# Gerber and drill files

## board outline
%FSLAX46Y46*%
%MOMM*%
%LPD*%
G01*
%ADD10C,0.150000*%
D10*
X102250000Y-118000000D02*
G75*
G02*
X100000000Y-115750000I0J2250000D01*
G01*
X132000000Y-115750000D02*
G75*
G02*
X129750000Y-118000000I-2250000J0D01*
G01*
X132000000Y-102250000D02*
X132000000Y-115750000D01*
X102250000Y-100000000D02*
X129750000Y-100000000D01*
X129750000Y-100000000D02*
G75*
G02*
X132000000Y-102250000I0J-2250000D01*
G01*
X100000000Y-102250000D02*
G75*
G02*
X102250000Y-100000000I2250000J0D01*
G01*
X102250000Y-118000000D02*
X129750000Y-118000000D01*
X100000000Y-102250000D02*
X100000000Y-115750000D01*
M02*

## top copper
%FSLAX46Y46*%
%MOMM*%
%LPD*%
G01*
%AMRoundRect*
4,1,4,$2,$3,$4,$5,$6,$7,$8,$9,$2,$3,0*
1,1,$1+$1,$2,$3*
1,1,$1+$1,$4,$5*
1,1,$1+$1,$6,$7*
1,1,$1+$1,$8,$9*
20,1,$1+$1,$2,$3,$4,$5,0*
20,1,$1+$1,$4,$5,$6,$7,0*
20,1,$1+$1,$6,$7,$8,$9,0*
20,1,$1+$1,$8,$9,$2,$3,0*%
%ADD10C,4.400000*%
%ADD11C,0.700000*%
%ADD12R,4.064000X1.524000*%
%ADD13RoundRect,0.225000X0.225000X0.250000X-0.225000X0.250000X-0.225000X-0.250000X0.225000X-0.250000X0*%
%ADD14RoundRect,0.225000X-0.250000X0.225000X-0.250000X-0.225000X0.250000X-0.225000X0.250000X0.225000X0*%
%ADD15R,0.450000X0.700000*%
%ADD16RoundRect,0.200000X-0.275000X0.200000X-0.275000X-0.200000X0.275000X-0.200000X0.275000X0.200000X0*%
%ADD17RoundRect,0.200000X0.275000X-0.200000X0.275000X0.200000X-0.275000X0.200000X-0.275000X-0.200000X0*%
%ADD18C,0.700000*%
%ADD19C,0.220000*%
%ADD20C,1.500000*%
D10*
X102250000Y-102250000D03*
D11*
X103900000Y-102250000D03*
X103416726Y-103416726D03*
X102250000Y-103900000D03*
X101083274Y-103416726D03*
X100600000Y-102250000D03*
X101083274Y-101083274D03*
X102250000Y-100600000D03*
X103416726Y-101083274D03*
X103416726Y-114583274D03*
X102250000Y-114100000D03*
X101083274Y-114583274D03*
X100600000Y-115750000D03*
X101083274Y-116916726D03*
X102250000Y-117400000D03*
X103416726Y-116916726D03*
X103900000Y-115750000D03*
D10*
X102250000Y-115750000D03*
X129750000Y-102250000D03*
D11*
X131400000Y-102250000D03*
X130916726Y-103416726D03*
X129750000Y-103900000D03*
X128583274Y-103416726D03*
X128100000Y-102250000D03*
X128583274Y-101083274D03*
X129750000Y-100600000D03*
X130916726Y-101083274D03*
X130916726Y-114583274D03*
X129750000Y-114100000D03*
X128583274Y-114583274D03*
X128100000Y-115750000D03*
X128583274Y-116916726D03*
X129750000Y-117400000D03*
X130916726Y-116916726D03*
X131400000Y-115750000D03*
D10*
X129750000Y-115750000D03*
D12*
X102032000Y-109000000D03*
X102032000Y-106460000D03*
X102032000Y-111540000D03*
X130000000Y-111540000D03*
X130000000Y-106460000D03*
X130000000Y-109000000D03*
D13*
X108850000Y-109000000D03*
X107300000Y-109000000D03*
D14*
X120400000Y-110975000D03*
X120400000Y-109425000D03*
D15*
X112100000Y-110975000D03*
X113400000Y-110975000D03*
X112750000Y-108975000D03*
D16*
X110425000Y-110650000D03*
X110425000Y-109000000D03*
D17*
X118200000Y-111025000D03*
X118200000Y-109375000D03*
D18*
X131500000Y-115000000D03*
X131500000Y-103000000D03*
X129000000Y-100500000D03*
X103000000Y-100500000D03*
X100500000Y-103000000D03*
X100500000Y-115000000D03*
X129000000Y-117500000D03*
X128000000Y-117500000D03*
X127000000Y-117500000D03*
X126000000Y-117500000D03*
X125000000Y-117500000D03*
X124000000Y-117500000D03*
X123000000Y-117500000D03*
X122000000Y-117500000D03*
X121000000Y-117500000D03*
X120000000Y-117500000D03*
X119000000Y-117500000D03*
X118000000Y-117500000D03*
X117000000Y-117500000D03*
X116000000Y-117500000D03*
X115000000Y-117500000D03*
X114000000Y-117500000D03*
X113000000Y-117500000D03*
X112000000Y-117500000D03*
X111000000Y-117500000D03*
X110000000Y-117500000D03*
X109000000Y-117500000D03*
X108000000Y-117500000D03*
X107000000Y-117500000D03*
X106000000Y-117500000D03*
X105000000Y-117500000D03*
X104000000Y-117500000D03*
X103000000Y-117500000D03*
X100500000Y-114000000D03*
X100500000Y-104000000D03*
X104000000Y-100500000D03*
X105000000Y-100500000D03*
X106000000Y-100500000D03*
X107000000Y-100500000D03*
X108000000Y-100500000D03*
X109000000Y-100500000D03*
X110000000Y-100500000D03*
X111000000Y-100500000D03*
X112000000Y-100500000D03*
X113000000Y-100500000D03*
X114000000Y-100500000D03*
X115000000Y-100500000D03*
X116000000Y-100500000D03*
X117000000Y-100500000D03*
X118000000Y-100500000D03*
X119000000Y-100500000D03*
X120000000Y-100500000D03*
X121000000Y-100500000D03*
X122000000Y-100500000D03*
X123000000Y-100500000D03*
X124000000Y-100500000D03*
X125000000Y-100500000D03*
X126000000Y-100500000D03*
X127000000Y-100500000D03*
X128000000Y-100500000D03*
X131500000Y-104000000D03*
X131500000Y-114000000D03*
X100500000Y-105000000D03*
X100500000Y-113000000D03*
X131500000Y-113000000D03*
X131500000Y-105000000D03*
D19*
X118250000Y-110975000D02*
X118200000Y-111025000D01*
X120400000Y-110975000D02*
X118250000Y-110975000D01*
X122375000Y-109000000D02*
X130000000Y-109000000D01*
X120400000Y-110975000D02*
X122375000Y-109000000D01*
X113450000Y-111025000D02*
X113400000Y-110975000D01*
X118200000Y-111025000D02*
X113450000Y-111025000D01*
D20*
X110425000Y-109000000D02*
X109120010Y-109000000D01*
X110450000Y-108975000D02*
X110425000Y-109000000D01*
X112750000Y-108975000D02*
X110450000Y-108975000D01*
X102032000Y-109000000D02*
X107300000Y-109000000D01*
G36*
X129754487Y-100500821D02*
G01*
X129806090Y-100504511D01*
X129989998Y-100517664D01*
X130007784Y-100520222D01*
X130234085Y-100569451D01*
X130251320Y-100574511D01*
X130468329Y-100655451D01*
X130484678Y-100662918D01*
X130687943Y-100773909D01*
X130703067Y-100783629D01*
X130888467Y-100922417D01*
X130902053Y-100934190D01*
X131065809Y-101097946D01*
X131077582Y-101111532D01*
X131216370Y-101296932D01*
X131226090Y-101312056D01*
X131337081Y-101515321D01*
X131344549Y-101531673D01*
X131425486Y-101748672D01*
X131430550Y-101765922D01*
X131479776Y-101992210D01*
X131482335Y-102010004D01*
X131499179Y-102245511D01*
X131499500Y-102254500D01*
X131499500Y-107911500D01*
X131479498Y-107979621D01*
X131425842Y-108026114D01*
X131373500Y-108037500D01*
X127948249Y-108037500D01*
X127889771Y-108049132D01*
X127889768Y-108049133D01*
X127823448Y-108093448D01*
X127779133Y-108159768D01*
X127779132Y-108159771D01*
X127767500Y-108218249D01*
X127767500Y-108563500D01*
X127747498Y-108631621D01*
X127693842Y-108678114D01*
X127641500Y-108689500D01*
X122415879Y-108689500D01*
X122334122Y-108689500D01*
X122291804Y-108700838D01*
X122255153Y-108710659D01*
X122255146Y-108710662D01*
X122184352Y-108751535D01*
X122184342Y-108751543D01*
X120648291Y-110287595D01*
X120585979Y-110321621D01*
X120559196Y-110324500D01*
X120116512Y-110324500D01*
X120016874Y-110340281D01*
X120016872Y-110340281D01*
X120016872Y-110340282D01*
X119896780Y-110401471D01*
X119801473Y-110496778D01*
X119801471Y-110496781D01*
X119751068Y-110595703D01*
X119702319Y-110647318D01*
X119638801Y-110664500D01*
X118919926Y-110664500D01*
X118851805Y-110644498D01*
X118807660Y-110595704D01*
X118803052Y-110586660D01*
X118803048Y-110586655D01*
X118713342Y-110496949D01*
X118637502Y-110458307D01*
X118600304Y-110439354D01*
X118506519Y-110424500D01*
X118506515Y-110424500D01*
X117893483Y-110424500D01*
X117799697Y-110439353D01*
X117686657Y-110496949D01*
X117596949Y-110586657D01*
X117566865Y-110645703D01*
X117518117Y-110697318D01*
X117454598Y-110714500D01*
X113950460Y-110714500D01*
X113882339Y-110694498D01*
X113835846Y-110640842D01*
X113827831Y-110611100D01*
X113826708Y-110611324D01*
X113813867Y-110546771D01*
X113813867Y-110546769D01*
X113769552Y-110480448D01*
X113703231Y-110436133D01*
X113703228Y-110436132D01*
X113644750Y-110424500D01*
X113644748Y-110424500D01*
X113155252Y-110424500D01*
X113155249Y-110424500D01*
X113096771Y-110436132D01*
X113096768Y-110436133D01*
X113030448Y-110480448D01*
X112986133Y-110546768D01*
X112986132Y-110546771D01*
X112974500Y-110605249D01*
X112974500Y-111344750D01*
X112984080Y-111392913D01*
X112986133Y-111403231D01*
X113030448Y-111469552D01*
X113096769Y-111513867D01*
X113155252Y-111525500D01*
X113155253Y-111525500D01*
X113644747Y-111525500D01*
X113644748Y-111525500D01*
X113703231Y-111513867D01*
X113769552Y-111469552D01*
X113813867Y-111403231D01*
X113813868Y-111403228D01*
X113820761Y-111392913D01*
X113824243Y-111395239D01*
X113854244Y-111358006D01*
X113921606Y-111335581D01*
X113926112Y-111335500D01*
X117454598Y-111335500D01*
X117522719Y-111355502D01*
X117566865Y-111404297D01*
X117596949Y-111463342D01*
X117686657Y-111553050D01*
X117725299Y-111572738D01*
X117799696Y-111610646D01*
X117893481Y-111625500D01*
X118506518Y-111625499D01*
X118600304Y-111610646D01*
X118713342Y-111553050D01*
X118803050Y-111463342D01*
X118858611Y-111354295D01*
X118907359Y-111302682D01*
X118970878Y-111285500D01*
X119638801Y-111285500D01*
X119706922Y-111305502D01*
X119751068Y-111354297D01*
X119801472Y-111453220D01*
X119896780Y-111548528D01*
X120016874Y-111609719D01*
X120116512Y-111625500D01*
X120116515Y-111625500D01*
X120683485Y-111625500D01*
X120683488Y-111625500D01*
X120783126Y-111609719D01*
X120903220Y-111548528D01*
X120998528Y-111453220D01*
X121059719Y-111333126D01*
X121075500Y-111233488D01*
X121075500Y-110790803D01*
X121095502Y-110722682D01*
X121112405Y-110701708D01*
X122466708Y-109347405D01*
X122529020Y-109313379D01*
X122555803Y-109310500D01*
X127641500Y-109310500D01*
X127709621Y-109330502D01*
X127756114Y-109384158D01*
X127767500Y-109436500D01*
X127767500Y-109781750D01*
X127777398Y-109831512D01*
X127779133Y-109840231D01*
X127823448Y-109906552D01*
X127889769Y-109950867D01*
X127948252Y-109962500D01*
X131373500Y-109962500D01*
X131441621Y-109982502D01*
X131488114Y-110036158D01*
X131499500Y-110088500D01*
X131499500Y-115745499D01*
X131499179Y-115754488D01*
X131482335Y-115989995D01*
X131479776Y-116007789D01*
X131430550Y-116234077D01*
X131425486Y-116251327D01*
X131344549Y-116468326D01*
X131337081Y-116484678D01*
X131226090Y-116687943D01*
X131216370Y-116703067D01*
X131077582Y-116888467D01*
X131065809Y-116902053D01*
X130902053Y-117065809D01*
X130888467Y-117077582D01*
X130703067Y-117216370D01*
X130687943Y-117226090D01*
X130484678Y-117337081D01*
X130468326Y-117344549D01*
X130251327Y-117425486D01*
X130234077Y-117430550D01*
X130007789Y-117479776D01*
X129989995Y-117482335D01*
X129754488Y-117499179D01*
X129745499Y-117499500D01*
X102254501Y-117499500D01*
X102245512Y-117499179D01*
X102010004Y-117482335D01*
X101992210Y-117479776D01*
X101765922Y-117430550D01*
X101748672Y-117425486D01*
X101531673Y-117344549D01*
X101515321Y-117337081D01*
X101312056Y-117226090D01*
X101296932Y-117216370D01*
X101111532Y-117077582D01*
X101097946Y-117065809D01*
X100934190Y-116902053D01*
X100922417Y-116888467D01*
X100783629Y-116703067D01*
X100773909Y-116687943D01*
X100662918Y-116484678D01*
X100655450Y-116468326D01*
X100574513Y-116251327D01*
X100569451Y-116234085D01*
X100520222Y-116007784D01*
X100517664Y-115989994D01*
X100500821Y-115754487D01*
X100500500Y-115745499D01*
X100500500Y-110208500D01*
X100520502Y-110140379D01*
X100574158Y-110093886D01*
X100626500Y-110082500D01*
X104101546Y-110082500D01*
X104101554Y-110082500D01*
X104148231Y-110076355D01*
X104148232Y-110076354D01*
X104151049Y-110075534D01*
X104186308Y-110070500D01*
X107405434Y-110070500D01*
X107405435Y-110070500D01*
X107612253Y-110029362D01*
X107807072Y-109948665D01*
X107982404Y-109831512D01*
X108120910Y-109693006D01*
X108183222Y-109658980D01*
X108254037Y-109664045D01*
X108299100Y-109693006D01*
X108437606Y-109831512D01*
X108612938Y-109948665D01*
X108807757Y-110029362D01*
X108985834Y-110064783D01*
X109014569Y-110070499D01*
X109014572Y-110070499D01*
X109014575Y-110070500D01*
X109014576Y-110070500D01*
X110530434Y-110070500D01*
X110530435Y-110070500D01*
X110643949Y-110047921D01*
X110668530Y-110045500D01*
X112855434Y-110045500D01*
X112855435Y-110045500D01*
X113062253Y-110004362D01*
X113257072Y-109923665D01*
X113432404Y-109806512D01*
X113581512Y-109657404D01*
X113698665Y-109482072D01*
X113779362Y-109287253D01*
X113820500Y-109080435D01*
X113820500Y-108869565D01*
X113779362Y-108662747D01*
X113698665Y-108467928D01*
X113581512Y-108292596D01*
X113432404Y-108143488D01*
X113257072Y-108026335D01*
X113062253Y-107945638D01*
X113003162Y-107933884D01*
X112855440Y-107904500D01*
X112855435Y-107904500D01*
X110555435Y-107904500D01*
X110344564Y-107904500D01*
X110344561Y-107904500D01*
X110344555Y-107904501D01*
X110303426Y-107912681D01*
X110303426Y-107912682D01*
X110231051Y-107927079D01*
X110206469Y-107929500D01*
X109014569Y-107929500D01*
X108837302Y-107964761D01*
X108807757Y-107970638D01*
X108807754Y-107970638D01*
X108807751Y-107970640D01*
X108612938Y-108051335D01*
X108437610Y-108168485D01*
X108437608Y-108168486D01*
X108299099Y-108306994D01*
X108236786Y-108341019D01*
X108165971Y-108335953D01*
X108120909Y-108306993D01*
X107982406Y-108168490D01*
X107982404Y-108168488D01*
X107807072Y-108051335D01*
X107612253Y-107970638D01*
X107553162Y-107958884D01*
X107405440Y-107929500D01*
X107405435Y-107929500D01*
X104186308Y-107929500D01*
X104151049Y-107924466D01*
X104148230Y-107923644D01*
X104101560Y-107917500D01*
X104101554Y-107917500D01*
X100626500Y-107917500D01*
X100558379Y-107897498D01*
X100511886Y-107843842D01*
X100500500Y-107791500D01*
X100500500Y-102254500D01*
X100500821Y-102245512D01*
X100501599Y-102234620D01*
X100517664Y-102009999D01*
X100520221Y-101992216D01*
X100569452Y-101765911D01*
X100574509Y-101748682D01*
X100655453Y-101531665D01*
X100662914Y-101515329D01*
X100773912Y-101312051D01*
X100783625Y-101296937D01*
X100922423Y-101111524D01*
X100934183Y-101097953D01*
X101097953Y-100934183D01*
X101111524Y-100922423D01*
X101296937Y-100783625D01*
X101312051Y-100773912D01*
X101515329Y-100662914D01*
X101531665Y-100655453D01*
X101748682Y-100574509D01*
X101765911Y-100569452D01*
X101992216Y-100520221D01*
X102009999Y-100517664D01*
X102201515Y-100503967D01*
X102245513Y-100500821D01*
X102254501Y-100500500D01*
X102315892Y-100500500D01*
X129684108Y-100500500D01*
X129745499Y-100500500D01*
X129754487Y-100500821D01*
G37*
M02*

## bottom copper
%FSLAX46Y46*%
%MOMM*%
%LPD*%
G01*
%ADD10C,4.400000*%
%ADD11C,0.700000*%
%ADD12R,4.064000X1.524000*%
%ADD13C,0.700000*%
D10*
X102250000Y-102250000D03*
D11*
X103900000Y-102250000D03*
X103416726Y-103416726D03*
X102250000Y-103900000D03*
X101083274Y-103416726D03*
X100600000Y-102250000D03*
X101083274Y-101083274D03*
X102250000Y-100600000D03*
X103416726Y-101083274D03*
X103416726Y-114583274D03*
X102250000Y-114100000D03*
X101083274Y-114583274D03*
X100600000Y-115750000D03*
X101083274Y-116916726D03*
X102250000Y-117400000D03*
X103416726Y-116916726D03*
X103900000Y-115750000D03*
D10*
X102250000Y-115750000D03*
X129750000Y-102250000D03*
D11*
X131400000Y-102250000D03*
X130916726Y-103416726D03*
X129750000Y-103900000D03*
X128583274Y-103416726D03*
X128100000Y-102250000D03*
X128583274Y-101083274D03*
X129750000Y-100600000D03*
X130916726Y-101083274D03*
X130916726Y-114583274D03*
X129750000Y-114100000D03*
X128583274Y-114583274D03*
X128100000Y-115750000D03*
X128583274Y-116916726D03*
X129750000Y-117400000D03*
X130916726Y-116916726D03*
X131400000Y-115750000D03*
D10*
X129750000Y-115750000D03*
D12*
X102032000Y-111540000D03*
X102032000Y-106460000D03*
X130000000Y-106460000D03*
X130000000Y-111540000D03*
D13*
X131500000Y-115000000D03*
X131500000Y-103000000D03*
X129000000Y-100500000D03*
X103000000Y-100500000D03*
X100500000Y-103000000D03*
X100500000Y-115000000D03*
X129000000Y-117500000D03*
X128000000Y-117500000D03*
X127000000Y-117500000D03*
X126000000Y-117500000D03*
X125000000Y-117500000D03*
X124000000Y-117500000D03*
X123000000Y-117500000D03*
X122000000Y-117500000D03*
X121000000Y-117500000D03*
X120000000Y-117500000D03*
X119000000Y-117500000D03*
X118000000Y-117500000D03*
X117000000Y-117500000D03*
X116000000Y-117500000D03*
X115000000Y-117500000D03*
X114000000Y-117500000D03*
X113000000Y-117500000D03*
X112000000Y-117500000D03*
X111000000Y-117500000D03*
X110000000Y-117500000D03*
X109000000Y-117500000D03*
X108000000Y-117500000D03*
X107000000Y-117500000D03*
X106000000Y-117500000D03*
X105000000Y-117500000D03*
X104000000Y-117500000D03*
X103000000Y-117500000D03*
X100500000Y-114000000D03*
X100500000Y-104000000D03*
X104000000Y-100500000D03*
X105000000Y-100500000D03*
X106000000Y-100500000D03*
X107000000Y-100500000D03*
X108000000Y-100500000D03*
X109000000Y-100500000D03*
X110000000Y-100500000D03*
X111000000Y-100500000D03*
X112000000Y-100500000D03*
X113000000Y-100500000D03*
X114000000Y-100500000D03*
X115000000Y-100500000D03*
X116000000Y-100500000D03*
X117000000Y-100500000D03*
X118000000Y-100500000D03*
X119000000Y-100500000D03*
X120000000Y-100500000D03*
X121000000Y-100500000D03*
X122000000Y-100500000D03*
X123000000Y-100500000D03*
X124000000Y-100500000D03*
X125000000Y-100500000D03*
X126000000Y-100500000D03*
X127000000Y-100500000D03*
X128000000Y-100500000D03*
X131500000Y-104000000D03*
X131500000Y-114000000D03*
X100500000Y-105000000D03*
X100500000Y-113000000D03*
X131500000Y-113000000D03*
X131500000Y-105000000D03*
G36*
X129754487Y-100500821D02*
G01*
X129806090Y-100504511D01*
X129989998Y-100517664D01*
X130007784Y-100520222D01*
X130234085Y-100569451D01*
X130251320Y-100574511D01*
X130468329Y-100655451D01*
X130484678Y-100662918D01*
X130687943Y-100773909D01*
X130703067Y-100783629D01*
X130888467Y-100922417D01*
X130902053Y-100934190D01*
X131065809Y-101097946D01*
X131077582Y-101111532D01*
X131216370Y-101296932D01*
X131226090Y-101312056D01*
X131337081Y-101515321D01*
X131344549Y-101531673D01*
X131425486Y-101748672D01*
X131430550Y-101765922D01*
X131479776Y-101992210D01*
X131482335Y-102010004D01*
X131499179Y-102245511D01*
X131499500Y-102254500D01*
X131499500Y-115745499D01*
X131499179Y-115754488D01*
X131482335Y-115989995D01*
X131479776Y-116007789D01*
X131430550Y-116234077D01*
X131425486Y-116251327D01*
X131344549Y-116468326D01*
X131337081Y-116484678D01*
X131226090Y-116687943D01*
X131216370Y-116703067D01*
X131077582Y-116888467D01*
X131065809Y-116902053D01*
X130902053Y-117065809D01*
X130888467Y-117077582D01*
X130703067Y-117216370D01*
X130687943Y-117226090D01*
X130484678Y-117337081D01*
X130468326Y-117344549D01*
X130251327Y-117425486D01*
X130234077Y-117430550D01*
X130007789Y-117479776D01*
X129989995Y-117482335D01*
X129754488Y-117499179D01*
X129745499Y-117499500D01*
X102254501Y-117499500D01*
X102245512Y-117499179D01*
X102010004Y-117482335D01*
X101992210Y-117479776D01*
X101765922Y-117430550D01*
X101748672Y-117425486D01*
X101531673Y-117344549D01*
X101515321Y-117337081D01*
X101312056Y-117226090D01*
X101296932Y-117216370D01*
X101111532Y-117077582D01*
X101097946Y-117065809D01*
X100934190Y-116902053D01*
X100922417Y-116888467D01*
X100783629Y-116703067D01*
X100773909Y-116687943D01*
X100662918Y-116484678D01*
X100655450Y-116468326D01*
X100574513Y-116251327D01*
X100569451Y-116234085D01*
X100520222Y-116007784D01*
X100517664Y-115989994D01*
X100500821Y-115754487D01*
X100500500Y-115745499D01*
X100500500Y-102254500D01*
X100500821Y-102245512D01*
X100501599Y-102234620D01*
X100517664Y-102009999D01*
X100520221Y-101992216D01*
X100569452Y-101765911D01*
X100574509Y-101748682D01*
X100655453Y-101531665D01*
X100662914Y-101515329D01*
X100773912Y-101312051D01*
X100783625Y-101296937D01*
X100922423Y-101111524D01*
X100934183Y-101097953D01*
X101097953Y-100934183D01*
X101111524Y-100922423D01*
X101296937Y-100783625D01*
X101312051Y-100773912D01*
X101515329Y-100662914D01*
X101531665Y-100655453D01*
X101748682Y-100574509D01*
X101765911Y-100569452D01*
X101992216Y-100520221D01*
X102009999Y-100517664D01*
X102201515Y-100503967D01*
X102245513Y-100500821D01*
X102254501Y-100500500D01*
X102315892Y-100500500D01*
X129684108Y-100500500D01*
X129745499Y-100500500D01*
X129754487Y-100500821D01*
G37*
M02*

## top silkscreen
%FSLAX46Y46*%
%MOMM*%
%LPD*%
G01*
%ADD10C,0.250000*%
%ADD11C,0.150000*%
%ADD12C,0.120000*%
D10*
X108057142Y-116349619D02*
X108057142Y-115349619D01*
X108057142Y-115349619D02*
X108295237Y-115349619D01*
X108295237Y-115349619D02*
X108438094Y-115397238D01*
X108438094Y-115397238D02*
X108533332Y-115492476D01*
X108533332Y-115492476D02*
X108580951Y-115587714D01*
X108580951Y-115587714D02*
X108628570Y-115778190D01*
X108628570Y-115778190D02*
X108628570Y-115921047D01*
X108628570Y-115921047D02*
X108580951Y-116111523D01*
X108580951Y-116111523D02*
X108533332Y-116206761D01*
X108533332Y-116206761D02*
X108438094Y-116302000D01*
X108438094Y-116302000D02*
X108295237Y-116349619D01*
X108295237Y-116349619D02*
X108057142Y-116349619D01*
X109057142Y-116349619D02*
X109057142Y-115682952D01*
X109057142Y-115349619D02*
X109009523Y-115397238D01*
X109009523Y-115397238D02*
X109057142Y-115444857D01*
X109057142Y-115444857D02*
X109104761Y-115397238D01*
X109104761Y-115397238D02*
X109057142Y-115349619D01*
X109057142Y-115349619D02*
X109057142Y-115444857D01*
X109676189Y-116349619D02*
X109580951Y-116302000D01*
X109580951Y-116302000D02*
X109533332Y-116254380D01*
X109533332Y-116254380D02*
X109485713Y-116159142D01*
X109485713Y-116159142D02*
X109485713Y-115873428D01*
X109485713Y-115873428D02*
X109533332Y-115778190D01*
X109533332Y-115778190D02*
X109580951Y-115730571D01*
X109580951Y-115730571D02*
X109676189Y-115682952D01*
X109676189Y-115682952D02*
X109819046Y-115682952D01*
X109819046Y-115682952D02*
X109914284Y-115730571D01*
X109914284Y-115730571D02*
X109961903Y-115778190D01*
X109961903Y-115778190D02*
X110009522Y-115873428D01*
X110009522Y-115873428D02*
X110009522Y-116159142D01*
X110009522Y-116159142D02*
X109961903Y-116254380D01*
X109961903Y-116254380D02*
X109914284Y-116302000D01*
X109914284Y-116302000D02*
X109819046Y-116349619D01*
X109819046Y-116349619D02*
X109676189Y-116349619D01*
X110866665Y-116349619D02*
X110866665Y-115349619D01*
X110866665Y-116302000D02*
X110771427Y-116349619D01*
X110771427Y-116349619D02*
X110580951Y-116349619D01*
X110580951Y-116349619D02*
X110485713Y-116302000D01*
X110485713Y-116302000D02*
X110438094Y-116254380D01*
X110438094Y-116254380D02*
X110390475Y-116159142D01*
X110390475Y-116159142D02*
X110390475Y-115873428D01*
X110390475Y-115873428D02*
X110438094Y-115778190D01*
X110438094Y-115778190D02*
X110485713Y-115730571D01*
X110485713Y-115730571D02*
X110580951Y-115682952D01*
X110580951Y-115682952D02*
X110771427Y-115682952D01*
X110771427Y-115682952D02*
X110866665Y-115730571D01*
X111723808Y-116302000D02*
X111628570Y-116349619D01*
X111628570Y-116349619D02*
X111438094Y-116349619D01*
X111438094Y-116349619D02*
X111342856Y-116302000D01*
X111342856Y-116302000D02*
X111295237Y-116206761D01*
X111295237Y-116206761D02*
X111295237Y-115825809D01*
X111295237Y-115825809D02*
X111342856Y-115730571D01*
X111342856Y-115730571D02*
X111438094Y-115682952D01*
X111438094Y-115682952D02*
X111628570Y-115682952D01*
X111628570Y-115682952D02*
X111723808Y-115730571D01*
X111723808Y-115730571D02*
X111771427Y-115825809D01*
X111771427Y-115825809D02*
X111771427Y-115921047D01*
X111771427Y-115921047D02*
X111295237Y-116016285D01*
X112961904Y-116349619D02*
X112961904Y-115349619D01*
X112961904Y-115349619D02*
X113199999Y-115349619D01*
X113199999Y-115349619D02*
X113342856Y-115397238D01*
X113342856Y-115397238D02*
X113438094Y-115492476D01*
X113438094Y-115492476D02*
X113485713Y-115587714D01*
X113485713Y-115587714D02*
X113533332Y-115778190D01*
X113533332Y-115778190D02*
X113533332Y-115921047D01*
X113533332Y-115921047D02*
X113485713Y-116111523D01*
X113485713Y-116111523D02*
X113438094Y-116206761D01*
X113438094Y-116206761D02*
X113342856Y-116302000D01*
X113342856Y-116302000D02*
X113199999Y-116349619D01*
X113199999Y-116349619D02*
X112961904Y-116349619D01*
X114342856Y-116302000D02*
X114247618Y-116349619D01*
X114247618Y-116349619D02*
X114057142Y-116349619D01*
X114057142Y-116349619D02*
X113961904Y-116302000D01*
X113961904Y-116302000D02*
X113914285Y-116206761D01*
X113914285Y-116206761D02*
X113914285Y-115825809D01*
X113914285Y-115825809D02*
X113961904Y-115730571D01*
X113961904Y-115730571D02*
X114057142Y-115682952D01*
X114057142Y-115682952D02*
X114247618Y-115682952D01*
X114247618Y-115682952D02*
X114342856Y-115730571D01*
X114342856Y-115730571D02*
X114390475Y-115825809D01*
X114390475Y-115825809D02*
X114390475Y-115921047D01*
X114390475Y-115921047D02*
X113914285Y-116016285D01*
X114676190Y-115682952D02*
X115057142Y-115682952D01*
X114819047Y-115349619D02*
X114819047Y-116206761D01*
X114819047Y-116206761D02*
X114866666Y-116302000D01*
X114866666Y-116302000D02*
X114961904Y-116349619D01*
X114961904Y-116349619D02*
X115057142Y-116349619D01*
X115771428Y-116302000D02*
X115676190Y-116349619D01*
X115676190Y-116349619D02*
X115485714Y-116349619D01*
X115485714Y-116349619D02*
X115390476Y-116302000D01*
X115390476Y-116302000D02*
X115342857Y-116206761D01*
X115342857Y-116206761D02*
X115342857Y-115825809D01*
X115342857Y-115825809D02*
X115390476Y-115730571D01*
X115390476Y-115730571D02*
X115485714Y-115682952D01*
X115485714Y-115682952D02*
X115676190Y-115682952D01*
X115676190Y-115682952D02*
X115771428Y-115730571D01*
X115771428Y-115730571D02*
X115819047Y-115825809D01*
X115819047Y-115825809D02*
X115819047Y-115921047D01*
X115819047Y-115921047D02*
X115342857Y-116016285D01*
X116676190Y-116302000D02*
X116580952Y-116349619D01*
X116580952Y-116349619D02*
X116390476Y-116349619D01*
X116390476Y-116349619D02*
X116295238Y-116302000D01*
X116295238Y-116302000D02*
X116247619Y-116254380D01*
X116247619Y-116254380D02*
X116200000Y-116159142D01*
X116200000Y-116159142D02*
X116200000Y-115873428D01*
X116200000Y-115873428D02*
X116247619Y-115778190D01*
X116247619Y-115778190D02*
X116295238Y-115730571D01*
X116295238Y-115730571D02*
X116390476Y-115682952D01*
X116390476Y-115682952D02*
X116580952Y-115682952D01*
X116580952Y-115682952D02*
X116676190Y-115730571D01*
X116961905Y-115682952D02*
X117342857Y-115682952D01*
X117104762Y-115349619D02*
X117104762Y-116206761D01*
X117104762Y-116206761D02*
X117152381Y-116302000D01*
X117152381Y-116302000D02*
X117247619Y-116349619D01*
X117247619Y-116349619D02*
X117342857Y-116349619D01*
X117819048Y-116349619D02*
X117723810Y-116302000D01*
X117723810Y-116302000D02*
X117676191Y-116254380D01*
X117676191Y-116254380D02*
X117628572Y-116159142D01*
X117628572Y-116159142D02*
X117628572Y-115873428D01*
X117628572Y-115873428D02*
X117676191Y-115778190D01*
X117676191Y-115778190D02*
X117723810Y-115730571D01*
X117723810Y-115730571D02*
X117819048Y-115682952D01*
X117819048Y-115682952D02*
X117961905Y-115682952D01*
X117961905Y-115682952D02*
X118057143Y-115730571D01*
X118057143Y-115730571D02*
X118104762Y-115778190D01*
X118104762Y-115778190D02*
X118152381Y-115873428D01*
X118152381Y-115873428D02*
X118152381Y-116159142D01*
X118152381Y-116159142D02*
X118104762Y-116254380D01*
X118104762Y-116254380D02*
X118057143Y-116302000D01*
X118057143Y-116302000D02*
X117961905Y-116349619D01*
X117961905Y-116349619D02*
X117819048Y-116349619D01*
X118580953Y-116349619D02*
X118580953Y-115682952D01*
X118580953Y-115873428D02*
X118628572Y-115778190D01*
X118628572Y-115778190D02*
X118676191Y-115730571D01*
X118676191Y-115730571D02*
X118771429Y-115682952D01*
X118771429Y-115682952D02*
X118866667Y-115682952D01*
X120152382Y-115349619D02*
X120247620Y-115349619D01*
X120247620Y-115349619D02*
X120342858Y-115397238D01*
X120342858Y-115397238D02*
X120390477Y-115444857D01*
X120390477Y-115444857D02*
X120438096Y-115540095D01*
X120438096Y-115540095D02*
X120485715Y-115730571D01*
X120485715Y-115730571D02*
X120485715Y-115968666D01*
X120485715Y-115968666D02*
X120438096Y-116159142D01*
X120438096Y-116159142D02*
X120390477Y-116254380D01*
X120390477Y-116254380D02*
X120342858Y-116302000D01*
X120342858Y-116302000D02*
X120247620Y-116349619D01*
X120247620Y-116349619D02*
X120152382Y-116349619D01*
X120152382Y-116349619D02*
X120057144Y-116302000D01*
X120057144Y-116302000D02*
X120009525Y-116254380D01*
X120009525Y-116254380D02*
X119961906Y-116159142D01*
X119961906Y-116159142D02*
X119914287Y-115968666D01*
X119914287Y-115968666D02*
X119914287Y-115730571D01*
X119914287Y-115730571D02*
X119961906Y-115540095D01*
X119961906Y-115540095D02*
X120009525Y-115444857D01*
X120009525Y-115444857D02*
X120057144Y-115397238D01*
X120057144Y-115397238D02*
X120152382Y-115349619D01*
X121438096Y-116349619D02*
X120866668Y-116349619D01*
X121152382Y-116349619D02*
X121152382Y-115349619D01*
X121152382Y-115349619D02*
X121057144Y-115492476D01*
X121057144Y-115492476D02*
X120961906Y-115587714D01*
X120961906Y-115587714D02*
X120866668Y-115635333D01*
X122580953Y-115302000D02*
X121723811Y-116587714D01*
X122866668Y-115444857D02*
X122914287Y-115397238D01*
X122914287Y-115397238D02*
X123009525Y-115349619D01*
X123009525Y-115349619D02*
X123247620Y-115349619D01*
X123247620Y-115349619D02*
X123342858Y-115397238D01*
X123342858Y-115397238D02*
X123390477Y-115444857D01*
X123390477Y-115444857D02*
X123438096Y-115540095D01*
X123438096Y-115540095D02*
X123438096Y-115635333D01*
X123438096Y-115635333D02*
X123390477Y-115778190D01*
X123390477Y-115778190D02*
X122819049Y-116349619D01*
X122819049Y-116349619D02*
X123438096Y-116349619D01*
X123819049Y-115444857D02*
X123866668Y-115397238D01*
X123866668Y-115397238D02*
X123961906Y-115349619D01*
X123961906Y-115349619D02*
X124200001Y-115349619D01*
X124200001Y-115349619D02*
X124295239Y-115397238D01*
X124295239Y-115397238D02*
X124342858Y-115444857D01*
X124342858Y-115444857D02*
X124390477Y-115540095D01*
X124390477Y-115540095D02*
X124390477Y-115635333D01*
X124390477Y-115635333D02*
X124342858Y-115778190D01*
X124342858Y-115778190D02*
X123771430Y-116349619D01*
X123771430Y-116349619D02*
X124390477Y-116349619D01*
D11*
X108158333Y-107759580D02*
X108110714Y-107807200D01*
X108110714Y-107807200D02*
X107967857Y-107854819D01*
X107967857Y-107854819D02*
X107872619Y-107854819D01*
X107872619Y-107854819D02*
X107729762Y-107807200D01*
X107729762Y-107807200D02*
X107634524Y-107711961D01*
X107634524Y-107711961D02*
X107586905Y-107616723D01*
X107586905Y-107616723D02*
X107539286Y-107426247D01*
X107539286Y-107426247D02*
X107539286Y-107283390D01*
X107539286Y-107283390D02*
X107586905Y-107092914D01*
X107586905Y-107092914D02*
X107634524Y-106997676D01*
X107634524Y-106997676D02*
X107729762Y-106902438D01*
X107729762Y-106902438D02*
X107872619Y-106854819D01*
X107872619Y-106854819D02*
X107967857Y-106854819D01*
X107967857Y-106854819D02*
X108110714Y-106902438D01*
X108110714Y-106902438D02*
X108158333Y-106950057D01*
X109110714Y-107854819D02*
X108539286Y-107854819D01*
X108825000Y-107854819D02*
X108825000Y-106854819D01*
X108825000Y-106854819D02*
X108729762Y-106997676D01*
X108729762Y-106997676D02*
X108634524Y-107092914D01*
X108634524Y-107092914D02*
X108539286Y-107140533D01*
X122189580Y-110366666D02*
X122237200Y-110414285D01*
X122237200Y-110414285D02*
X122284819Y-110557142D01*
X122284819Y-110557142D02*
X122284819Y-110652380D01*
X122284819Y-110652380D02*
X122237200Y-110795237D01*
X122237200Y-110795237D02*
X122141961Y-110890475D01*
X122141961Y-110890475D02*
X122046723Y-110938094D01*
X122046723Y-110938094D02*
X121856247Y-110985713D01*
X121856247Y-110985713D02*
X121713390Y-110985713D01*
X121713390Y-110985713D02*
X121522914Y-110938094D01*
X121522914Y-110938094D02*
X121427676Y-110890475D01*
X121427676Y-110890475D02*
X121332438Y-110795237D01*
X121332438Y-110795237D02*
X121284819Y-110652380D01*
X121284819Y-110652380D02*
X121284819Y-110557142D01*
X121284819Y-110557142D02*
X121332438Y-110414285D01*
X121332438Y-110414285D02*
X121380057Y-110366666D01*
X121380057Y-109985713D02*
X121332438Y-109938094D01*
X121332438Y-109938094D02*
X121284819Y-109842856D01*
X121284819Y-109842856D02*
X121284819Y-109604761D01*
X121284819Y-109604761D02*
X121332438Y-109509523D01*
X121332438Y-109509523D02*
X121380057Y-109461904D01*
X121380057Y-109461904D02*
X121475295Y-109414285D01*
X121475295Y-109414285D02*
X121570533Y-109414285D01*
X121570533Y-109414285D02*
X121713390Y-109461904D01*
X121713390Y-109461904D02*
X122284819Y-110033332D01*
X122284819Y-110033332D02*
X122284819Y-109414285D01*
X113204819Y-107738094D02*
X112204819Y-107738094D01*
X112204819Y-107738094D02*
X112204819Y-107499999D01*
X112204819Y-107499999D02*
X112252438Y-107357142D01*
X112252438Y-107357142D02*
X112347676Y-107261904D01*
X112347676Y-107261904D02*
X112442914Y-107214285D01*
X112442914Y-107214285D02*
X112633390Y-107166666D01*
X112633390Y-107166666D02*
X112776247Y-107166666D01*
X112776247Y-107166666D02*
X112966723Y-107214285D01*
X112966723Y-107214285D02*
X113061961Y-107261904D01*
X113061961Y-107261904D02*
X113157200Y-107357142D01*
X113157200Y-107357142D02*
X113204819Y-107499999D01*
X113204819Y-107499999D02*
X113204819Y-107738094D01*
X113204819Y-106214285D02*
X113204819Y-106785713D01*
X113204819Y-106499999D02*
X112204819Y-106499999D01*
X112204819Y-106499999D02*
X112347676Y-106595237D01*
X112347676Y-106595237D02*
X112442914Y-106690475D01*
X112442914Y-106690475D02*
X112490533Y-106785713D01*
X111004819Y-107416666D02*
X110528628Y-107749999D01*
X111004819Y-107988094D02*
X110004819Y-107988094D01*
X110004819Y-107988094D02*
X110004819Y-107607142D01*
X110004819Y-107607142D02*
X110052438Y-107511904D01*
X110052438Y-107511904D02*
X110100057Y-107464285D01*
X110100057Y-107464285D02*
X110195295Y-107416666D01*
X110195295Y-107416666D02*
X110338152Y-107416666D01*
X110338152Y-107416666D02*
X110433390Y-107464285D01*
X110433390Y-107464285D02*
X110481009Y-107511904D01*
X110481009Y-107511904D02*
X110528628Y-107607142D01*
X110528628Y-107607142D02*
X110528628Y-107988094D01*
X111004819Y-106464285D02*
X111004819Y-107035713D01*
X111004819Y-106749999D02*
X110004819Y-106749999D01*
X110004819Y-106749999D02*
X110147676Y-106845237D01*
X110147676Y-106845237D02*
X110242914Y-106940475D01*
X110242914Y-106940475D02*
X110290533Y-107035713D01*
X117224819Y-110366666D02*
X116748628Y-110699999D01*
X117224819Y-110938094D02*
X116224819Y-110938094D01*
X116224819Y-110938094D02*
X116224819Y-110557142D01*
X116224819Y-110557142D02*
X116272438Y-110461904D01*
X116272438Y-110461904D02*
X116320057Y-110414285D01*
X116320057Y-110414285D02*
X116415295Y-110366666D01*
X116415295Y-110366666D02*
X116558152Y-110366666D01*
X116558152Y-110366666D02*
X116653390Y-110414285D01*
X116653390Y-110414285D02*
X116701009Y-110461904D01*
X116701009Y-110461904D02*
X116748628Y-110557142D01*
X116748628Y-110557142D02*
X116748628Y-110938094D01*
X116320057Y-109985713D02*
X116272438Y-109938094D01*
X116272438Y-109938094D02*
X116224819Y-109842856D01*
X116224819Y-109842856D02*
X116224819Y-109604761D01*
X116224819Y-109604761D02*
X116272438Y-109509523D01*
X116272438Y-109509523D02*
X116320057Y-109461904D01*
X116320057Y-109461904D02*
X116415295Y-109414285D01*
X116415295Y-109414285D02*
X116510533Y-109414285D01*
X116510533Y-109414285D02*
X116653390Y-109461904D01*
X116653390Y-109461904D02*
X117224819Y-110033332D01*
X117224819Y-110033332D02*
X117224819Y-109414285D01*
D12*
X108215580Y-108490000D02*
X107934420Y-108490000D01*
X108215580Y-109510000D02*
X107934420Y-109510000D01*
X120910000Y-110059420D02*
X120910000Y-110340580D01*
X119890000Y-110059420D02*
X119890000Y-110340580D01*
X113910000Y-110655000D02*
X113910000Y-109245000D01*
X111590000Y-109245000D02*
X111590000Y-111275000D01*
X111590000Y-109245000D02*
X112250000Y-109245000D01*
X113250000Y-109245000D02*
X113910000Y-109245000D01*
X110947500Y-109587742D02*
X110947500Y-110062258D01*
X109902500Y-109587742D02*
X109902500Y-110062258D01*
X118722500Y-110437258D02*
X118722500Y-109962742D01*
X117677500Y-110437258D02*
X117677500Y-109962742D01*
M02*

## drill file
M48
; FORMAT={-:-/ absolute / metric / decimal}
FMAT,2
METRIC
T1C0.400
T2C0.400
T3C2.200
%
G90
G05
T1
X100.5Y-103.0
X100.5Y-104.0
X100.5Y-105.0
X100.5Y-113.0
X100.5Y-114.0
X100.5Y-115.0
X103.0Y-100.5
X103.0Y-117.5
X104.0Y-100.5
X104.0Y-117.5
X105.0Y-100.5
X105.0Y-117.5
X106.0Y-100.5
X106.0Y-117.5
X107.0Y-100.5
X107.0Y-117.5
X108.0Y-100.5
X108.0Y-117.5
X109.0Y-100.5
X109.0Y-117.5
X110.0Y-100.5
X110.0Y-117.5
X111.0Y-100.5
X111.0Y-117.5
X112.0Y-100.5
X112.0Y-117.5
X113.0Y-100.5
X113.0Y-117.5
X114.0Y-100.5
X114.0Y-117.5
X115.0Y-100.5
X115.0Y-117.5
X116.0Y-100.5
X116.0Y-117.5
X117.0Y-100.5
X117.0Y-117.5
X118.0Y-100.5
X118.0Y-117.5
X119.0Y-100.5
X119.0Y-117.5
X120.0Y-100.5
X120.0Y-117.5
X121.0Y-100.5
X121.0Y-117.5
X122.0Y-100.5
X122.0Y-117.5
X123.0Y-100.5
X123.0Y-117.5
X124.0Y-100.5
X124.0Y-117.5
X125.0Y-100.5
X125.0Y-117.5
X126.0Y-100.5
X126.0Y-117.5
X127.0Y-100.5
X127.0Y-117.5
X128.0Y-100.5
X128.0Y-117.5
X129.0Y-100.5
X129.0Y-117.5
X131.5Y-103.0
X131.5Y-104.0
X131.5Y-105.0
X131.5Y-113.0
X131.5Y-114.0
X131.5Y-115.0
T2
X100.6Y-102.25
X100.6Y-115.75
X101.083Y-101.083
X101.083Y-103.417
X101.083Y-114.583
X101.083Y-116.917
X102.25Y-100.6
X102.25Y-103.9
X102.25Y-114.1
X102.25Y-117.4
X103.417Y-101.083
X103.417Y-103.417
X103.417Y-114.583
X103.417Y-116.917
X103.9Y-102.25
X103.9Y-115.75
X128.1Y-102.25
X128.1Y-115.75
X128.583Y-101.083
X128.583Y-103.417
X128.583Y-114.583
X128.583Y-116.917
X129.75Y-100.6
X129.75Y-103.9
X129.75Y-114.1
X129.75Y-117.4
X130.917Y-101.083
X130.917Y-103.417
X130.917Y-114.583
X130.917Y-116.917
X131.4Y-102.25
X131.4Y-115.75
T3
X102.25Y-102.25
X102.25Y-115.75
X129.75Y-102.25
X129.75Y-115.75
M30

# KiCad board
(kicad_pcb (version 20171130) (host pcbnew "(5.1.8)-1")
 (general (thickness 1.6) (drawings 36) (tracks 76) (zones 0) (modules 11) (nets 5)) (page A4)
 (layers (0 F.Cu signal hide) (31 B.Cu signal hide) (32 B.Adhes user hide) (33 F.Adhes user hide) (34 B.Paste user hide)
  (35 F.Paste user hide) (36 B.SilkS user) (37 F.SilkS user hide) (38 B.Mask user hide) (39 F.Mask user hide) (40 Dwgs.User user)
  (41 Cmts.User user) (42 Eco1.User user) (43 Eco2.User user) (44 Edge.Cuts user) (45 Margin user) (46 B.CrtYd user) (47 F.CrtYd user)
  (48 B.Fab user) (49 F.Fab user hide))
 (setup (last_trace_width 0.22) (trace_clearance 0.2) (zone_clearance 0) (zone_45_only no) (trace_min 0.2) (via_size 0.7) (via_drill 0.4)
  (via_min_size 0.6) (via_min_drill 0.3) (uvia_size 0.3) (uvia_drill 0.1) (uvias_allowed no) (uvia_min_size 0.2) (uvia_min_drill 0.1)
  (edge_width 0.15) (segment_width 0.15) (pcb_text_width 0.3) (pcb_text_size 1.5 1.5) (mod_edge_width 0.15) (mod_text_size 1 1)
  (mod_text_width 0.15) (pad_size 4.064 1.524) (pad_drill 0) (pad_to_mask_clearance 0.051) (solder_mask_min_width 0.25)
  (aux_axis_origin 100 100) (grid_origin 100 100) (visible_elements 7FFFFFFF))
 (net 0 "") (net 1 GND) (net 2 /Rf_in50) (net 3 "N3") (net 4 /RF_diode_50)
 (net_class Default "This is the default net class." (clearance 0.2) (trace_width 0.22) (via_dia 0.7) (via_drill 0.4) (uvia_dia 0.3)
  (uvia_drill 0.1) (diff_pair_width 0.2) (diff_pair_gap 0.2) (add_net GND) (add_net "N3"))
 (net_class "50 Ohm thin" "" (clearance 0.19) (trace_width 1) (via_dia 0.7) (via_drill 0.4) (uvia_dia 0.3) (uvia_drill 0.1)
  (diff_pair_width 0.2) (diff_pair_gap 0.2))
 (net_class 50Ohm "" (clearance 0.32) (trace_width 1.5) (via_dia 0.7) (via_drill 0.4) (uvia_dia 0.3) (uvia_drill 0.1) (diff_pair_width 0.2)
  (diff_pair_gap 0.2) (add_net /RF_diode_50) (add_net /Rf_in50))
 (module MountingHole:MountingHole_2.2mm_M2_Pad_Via (layer F.Cu) (at 102.25 102.25)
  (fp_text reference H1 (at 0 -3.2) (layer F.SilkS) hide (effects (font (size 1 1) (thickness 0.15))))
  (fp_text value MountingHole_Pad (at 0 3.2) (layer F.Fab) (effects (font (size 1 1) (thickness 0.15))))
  (pad 1 thru_hole circle (at 0 0) (size 4.4 4.4) (drill 2.2) (layers *.Cu *.Mask) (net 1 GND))
  (pad 1 thru_hole circle (at 1.65 0) (size 0.7 0.7) (drill 0.4) (layers *.Cu *.Mask) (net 1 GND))
  (pad 1 thru_hole circle (at 1.166726 1.166726) (size 0.7 0.7) (drill 0.4) (layers *.Cu *.Mask) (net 1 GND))
  (pad 1 thru_hole circle (at 0 1.65) (size 0.7 0.7) (drill 0.4) (layers *.Cu *.Mask) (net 1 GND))
  (pad 1 thru_hole circle (at -1.166726 1.166726) (size 0.7 0.7) (drill 0.4) (layers *.Cu *.Mask) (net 1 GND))
  (pad 1 thru_hole circle (at -1.65 0) (size 0.7 0.7) (drill 0.4) (layers *.Cu *.Mask) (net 1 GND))
  (pad 1 thru_hole circle (at -1.166726 -1.166726) (size 0.7 0.7) (drill 0.4) (layers *.Cu *.Mask) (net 1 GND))
  (pad 1 thru_hole circle (at 0 -1.65) (size 0.7 0.7) (drill 0.4) (layers *.Cu *.Mask) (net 1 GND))
  (pad 1 thru_hole circle (at 1.166726 -1.166726) (size 0.7 0.7) (drill 0.4) (layers *.Cu *.Mask) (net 1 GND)))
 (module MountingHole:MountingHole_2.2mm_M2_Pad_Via (layer F.Cu) (at 102.25 115.75)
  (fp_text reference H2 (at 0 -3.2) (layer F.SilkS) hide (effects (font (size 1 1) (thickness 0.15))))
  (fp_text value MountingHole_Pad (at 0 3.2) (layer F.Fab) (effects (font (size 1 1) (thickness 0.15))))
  (pad 1 thru_hole circle (at 1.166726 -1.166726) (size 0.7 0.7) (drill 0.4) (layers *.Cu *.Mask) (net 1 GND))
  (pad 1 thru_hole circle (at 0 -1.65) (size 0.7 0.7) (drill 0.4) (layers *.Cu *.Mask) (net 1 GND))
  (pad 1 thru_hole circle (at -1.166726 -1.166726) (size 0.7 0.7) (drill 0.4) (layers *.Cu *.Mask) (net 1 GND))
  (pad 1 thru_hole circle (at -1.65 0) (size 0.7 0.7) (drill 0.4) (layers *.Cu *.Mask) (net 1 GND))
  (pad 1 thru_hole circle (at -1.166726 1.166726) (size 0.7 0.7) (drill 0.4) (layers *.Cu *.Mask) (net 1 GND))
  (pad 1 thru_hole circle (at 0 1.65) (size 0.7 0.7) (drill 0.4) (layers *.Cu *.Mask) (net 1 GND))
  (pad 1 thru_hole circle (at 1.166726 1.166726) (size 0.7 0.7) (drill 0.4) (layers *.Cu *.Mask) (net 1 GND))
  (pad 1 thru_hole circle (at 1.65 0) (size 0.7 0.7) (drill 0.4) (layers *.Cu *.Mask) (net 1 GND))
  (pad 1 thru_hole circle (at 0 0) (size 4.4 4.4) (drill 2.2) (layers *.Cu *.Mask) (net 1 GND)))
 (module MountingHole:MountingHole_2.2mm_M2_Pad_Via (layer F.Cu) (at 129.75 102.25)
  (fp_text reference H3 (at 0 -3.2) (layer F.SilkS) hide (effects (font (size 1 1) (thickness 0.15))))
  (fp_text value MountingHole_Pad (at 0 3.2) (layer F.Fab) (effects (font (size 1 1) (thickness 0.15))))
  (pad 1 thru_hole circle (at 0 0) (size 4.4 4.4) (drill 2.2) (layers *.Cu *.Mask) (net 1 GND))
  (pad 1 thru_hole circle (at 1.65 0) (size 0.7 0.7) (drill 0.4) (layers *.Cu *.Mask) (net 1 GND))
  (pad 1 thru_hole circle (at 1.166726 1.166726) (size 0.7 0.7) (drill 0.4) (layers *.Cu *.Mask) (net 1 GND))
  (pad 1 thru_hole circle (at 0 1.65) (size 0.7 0.7) (drill 0.4) (layers *.Cu *.Mask) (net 1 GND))
  (pad 1 thru_hole circle (at -1.166726 1.166726) (size 0.7 0.7) (drill 0.4) (layers *.Cu *.Mask) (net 1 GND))
  (pad 1 thru_hole circle (at -1.65 0) (size 0.7 0.7) (drill 0.4) (layers *.Cu *.Mask) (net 1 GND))
  (pad 1 thru_hole circle (at -1.166726 -1.166726) (size 0.7 0.7) (drill 0.4) (layers *.Cu *.Mask) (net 1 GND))
  (pad 1 thru_hole circle (at 0 -1.65) (size 0.7 0.7) (drill 0.4) (layers *.Cu *.Mask) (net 1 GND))
  (pad 1 thru_hole circle (at 1.166726 -1.166726) (size 0.7 0.7) (drill 0.4) (layers *.Cu *.Mask) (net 1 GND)))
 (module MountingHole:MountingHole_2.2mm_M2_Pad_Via (layer F.Cu) (at 129.75 115.75)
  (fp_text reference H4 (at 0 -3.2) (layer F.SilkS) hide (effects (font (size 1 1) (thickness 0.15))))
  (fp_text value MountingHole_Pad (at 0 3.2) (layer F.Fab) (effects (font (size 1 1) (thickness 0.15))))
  (pad 1 thru_hole circle (at 1.166726 -1.166726) (size 0.7 0.7) (drill 0.4) (layers *.Cu *.Mask) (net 1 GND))
  (pad 1 thru_hole circle (at 0 -1.65) (size 0.7 0.7) (drill 0.4) (layers *.Cu *.Mask) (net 1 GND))
  (pad 1 thru_hole circle (at -1.166726 -1.166726) (size 0.7 0.7) (drill 0.4) (layers *.Cu *.Mask) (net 1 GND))
  (pad 1 thru_hole circle (at -1.65 0) (size 0.7 0.7) (drill 0.4) (layers *.Cu *.Mask) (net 1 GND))
  (pad 1 thru_hole circle (at -1.166726 1.166726) (size 0.7 0.7) (drill 0.4) (layers *.Cu *.Mask) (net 1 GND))
  (pad 1 thru_hole circle (at 0 1.65) (size 0.7 0.7) (drill 0.4) (layers *.Cu *.Mask) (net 1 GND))
  (pad 1 thru_hole circle (at 1.166726 1.166726) (size 0.7 0.7) (drill 0.4) (layers *.Cu *.Mask) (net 1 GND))
  (pad 1 thru_hole circle (at 1.65 0) (size 0.7 0.7) (drill 0.4) (layers *.Cu *.Mask) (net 1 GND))
  (pad 1 thru_hole circle (at 0 0) (size 4.4 4.4) (drill 2.2) (layers *.Cu *.Mask) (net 1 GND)))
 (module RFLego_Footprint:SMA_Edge (layer F.Cu) (at 100 109)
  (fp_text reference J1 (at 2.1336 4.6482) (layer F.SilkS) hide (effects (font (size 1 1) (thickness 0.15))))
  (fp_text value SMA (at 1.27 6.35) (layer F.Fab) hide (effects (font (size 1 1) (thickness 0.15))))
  (pad 1 smd rect (at 2.032 0) (size 4.064 1.524) (layers F.Cu F.Mask) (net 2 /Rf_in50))
  (pad 2 smd rect (at 2.032 -2.54) (size 4.064 1.524) (layers F.Cu F.Mask) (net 1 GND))
  (pad 2 smd rect (at 2.032 2.54) (size 4.064 1.524) (layers B.Cu B.Mask) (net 1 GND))
  (pad 2 smd rect (at 2.032 -2.54) (size 4.064 1.524) (layers B.Cu B.Mask) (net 1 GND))
  (pad 2 smd rect (at 2.032 2.54) (size 4.064 1.524) (layers F.Cu F.Mask) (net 1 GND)))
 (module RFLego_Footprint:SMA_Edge (layer F.Cu) (at 127.968 109)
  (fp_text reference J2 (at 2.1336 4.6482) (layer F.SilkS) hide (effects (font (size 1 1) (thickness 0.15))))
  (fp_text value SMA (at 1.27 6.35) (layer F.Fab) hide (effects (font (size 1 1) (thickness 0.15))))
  (pad 2 smd rect (at 2.032 2.54) (size 4.064 1.524) (layers F.Cu F.Mask) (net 1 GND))
  (pad 2 smd rect (at 2.032 -2.54) (size 4.064 1.524) (layers B.Cu B.Mask) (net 1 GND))
  (pad 2 smd rect (at 2.032 2.54) (size 4.064 1.524) (layers B.Cu B.Mask) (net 1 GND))
  (pad 2 smd rect (at 2.032 -2.54) (size 4.064 1.524) (layers F.Cu F.Mask) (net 1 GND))
  (pad 1 smd rect (at 2.032 0) (size 4.064 1.524) (layers F.Cu F.Mask) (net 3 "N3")))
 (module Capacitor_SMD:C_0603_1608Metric (layer F.Cu) (at 108.075 109 180)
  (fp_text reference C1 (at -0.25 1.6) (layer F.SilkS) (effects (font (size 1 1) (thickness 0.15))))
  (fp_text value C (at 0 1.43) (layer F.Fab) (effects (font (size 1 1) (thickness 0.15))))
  (fp_line (start -0.14058 0.51) (end 0.14058 0.51) (layer F.SilkS) (width 0.12))
  (fp_line (start -0.14058 -0.51) (end 0.14058 -0.51) (layer F.SilkS) (width 0.12))
  (pad 1 smd roundrect (at -0.775 0 180) (size 0.9 0.95) (layers F.Cu F.Paste F.Mask) (roundrect_rratio 0.25) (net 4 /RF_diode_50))
  (pad 2 smd roundrect (at 0.775 0 180) (size 0.9 0.95) (layers F.Cu F.Paste F.Mask) (roundrect_rratio 0.25) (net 2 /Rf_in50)))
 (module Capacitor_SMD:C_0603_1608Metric (layer F.Cu) (at 120.4 110.2 270)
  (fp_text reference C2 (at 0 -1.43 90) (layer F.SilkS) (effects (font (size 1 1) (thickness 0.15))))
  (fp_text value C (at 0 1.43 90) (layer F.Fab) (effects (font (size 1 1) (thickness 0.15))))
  (fp_line (start -0.14058 -0.51) (end 0.14058 -0.51) (layer F.SilkS) (width 0.12))
  (fp_line (start -0.14058 0.51) (end 0.14058 0.51) (layer F.SilkS) (width 0.12))
  (pad 2 smd roundrect (at 0.775 0 270) (size 0.9 0.95) (layers F.Cu F.Paste F.Mask) (roundrect_rratio 0.25) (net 3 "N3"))
  (pad 1 smd roundrect (at -0.775 0 270) (size 0.9 0.95) (layers F.Cu F.Paste F.Mask) (roundrect_rratio 0.25) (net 1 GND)))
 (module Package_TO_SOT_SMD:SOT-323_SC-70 (layer F.Cu) (at 112.75 109.975 90)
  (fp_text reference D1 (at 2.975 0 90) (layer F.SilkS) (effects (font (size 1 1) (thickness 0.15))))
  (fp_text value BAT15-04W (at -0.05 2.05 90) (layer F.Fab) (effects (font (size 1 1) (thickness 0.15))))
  (fp_line (start -0.68 1.16) (end 0.73 1.16) (layer F.SilkS) (width 0.12))
  (fp_line (start 0.73 -1.16) (end -1.3 -1.16) (layer F.SilkS) (width 0.12))
  (fp_line (start 0.73 -1.16) (end 0.73 -0.5) (layer F.SilkS) (width 0.12))
  (fp_line (start 0.73 0.5) (end 0.73 1.16) (layer F.SilkS) (width 0.12))
  (pad 1 smd rect (at -1 -0.65) (size 0.45 0.7) (layers F.Cu F.Paste F.Mask) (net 1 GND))
  (pad 2 smd rect (at -1 0.65) (size 0.45 0.7) (layers F.Cu F.Paste F.Mask) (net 3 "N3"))
  (pad 3 smd rect (at 1 0) (size 0.45 0.7) (layers F.Cu F.Paste F.Mask) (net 4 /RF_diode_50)))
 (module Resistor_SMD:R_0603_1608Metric (layer F.Cu) (at 110.425 109.825 270)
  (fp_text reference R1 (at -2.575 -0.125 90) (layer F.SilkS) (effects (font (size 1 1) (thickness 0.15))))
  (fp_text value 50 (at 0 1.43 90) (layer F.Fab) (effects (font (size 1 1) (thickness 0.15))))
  (fp_line (start -0.237258 -0.5225) (end 0.237258 -0.5225) (layer F.SilkS) (width 0.12))
  (fp_line (start -0.237258 0.5225) (end 0.237258 0.5225) (layer F.SilkS) (width 0.12))
  (pad 2 smd roundrect (at 0.825 0 270) (size 0.8 0.95) (layers F.Cu F.Paste F.Mask) (roundrect_rratio 0.25) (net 1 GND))
  (pad 1 smd roundrect (at -0.825 0 270) (size 0.8 0.95) (layers F.Cu F.Paste F.Mask) (roundrect_rratio 0.25) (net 4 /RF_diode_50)))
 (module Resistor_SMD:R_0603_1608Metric (layer F.Cu) (at 118.2 110.2 90)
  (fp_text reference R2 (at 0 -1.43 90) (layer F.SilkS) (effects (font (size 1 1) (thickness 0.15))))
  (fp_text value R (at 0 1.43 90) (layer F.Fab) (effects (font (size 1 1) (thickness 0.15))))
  (fp_line (start -0.237258 0.5225) (end 0.237258 0.5225) (layer F.SilkS) (width 0.12))
  (fp_line (start -0.237258 -0.5225) (end 0.237258 -0.5225) (layer F.SilkS) (width 0.12))
  (pad 1 smd roundrect (at -0.825 0 90) (size 0.8 0.95) (layers F.Cu F.Paste F.Mask) (roundrect_rratio 0.25) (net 3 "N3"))
  (pad 2 smd roundrect (at 0.825 0 90) (size 0.8 0.95) (layers F.Cu F.Paste F.Mask) (roundrect_rratio 0.25) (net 1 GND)))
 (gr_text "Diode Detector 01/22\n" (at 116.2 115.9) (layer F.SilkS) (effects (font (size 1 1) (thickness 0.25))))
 (gr_arc (start 102.25 115.75) (end 100 115.75) (angle -90) (layer Edge.Cuts) (width 0.15))
 (gr_arc (start 129.75 115.75) (end 129.75 118) (angle -90) (layer Edge.Cuts) (width 0.15))
 (gr_line (start 132 102.25) (end 132 115.75) (layer Edge.Cuts) (width 0.15))
 (gr_line (start 102.25 100) (end 129.75 100) (layer Edge.Cuts) (width 0.15))
 (gr_arc (start 129.75 102.25) (end 132 102.25) (angle -90) (layer Edge.Cuts) (width 0.15))
 (gr_arc (start 102.25 102.25) (end 102.25 100) (angle -90) (layer Edge.Cuts) (width 0.15))
 (gr_line (start 102.25 118) (end 129.75 118) (layer Edge.Cuts) (width 0.15))
 (gr_line (start 100 102.25) (end 100 115.75) (layer Edge.Cuts) (width 0.15))
 (via (at 131.5 115) (size 0.7) (drill 0.4) (layers F.Cu B.Cu) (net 1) (status 30))
 (via (at 131.5 103) (size 0.7) (drill 0.4) (layers F.Cu B.Cu) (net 1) (status 30))
 (via (at 129 100.5) (size 0.7) (drill 0.4) (layers F.Cu B.Cu) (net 1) (status 30))
 (via (at 103 100.5) (size 0.7) (drill 0.4) (layers F.Cu B.Cu) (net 1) (status 30))
 (via (at 100.5 103) (size 0.7) (drill 0.4) (layers F.Cu B.Cu) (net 1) (status 30))
 (via (at 100.5 115) (size 0.7) (drill 0.4) (layers F.Cu B.Cu) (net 1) (status 30))
 (via (at 129 117.5) (size 0.7) (drill 0.4) (layers F.Cu B.Cu) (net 1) (status 30))
 (via (at 128 117.5) (size 0.7) (drill 0.4) (layers F.Cu B.Cu) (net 1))
 (via (at 127 117.5) (size 0.7) (drill 0.4) (layers F.Cu B.Cu) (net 1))
 (via (at 126 117.5) (size 0.7) (drill 0.4) (layers F.Cu B.Cu) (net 1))
 (via (at 125 117.5) (size 0.7) (drill 0.4) (layers F.Cu B.Cu) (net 1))
 (via (at 124 117.5) (size 0.7) (drill 0.4) (layers F.Cu B.Cu) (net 1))
 (via (at 123 117.5) (size 0.7) (drill 0.4) (layers F.Cu B.Cu) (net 1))
 (via (at 122 117.5) (size 0.7) (drill 0.4) (layers F.Cu B.Cu) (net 1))
 (via (at 121 117.5) (size 0.7) (drill 0.4) (layers F.Cu B.Cu) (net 1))
 (via (at 120 117.5) (size 0.7) (drill 0.4) (layers F.Cu B.Cu) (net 1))
 (via (at 119 117.5) (size 0.7) (drill 0.4) (layers F.Cu B.Cu) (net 1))
 (via (at 118 117.5) (size 0.7) (drill 0.4) (layers F.Cu B.Cu) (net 1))
 (via (at 117 117.5) (size 0.7) (drill 0.4) (layers F.Cu B.Cu) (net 1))
 (via (at 116 117.5) (size 0.7) (drill 0.4) (layers F.Cu B.Cu) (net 1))
 (via (at 115 117.5) (size 0.7) (drill 0.4) (layers F.Cu B.Cu) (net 1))
 (via (at 114 117.5) (size 0.7) (drill 0.4) (layers F.Cu B.Cu) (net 1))
 (via (at 113 117.5) (size 0.7) (drill 0.4) (layers F.Cu B.Cu) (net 1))
 (via (at 112 117.5) (size 0.7) (drill 0.4) (layers F.Cu B.Cu) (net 1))
 (via (at 111 117.5) (size 0.7) (drill 0.4) (layers F.Cu B.Cu) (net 1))
 (via (at 110 117.5) (size 0.7) (drill 0.4) (layers F.Cu B.Cu) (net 1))
 (via (at 109 117.5) (size 0.7) (drill 0.4) (layers F.Cu B.Cu) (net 1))
 (via (at 108 117.5) (size 0.7) (drill 0.4) (layers F.Cu B.Cu) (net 1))
 (via (at 107 117.5) (size 0.7) (drill 0.4) (layers F.Cu B.Cu) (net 1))
 (via (at 106 117.5) (size 0.7) (drill 0.4) (layers F.Cu B.Cu) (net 1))
 (via (at 105 117.5) (size 0.7) (drill 0.4) (layers F.Cu B.Cu) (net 1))
 (via (at 104 117.5) (size 0.7) (drill 0.4) (layers F.Cu B.Cu) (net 1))
 (via (at 103 117.5) (size 0.7) (drill 0.4) (layers F.Cu B.Cu) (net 1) (status 30))
 (via (at 100.5 114) (size 0.7) (drill 0.4) (layers F.Cu B.Cu) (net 1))
 (via (at 100.5 104) (size 0.7) (drill 0.4) (layers F.Cu B.Cu) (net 1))
 (via (at 104 100.5) (size 0.7) (drill 0.4) (layers F.Cu B.Cu) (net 1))
 (via (at 105 100.5) (size 0.7) (drill 0.4) (layers F.Cu B.Cu) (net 1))
 (via (at 106 100.5) (size 0.7) (drill 0.4) (layers F.Cu B.Cu) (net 1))
 (via (at 107 100.5) (size 0.7) (drill 0.4) (layers F.Cu B.Cu) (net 1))
 (via (at 108 100.5) (size 0.7) (drill 0.4) (layers F.Cu B.Cu) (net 1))
 (via (at 109 100.5) (size 0.7) (drill 0.4) (layers F.Cu B.Cu) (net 1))
 (via (at 110 100.5) (size 0.7) (drill 0.4) (layers F.Cu B.Cu) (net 1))
 (via (at 111 100.5) (size 0.7) (drill 0.4) (layers F.Cu B.Cu) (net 1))
 (via (at 112 100.5) (size 0.7) (drill 0.4) (layers F.Cu B.Cu) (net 1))
 (via (at 113 100.5) (size 0.7) (drill 0.4) (layers F.Cu B.Cu) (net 1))
 (via (at 114 100.5) (size 0.7) (drill 0.4) (layers F.Cu B.Cu) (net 1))
 (via (at 115 100.5) (size 0.7) (drill 0.4) (layers F.Cu B.Cu) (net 1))
 (via (at 116 100.5) (size 0.7) (drill 0.4) (layers F.Cu B.Cu) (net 1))
 (via (at 117 100.5) (size 0.7) (drill 0.4) (layers F.Cu B.Cu) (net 1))
 (via (at 118 100.5) (size 0.7) (drill 0.4) (layers F.Cu B.Cu) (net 1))
 (via (at 119 100.5) (size 0.7) (drill 0.4) (layers F.Cu B.Cu) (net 1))
 (via (at 120 100.5) (size 0.7) (drill 0.4) (layers F.Cu B.Cu) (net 1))
 (via (at 121 100.5) (size 0.7) (drill 0.4) (layers F.Cu B.Cu) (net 1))
 (via (at 122 100.5) (size 0.7) (drill 0.4) (layers F.Cu B.Cu) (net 1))
 (via (at 123 100.5) (size 0.7) (drill 0.4) (layers F.Cu B.Cu) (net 1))
 (via (at 124 100.5) (size 0.7) (drill 0.4) (layers F.Cu B.Cu) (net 1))
 (via (at 125 100.5) (size 0.7) (drill 0.4) (layers F.Cu B.Cu) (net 1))
 (via (at 126 100.5) (size 0.7) (drill 0.4) (layers F.Cu B.Cu) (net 1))
 (via (at 127 100.5) (size 0.7) (drill 0.4) (layers F.Cu B.Cu) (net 1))
 (via (at 128 100.5) (size 0.7) (drill 0.4) (layers F.Cu B.Cu) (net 1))
 (via (at 131.5 104) (size 0.7) (drill 0.4) (layers F.Cu B.Cu) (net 1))
 (via (at 131.5 114) (size 0.7) (drill 0.4) (layers F.Cu B.Cu) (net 1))
 (via (at 100.5 105) (size 0.7) (drill 0.4) (layers F.Cu B.Cu) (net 1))
 (via (at 100.5 113) (size 0.7) (drill 0.4) (layers F.Cu B.Cu) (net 1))
 (via (at 131.5 113) (size 0.7) (drill 0.4) (layers F.Cu B.Cu) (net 1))
 (via (at 131.5 105) (size 0.7) (drill 0.4) (layers F.Cu B.Cu) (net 1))
 (segment (start 118.25 110.975) (end 118.2 111.025) (width 0.22) (layer F.Cu) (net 3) (status 30))
 (segment (start 120.4 110.975) (end 118.25 110.975) (width 0.22) (layer F.Cu) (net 3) (status 30))
 (segment (start 122.375 109) (end 130 109) (width 0.22) (layer F.Cu) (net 3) (status 20))
 (segment (start 120.4 110.975) (end 122.375 109) (width 0.22) (layer F.Cu) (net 3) (status 10))
 (segment (start 113.45 111.025) (end 113.4 110.975) (width 0.22) (layer F.Cu) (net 3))
 (segment (start 118.2 111.025) (end 113.45 111.025) (width 0.22) (layer F.Cu) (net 3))
 (segment (start 110.425 109) (end 109.12001 109) (width 1.5) (layer F.Cu) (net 4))
 (segment (start 110.45 108.975) (end 110.425 109) (width 1.5) (layer F.Cu) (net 4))
 (segment (start 112.75 108.975) (end 110.45 108.975) (width 1.5) (layer F.Cu) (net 4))
 (segment (start 102.032 109) (end 107.3 109) (width 1.5) (layer F.Cu) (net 2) (status 30))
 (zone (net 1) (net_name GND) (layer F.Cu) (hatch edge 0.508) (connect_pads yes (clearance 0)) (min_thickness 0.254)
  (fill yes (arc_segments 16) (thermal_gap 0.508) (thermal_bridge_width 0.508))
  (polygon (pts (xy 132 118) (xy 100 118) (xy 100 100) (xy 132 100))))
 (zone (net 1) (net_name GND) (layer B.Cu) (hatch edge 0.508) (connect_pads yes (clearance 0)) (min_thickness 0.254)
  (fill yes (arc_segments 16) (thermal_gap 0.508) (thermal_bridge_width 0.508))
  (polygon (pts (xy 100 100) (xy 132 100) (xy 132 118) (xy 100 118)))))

